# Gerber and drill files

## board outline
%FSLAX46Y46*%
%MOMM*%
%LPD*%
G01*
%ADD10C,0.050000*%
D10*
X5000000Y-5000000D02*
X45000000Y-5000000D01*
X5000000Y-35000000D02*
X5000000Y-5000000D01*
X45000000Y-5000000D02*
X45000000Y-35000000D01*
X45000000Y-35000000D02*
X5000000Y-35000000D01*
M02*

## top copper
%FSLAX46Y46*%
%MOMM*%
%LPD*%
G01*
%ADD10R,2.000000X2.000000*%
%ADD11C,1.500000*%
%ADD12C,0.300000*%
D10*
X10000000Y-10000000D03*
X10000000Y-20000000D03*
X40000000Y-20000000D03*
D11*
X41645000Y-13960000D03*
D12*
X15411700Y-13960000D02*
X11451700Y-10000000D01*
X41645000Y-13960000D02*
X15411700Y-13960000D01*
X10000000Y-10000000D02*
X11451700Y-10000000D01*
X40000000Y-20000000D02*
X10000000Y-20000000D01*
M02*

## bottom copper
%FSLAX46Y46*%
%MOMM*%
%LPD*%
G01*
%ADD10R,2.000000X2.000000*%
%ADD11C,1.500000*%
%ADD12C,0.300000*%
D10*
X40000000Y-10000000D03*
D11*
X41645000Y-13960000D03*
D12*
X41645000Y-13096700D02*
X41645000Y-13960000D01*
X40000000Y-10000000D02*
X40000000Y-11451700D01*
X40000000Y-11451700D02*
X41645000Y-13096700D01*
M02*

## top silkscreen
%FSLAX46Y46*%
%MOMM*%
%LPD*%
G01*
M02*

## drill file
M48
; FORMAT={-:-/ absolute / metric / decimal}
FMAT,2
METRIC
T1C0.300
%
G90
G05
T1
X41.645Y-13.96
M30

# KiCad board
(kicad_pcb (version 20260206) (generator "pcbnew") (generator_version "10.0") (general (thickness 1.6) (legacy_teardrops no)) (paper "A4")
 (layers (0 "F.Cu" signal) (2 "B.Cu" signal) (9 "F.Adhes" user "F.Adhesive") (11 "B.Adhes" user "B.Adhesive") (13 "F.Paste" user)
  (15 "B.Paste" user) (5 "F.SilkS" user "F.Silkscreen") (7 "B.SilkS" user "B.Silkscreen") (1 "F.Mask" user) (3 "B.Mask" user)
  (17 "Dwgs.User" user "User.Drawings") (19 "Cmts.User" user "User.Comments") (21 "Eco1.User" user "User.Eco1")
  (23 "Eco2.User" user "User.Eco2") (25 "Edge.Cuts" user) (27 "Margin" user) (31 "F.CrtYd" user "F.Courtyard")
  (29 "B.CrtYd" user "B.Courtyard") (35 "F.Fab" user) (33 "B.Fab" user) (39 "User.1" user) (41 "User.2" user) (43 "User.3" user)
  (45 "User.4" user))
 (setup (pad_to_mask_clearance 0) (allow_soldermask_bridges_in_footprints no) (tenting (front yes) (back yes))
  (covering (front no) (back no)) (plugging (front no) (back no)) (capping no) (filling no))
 (gr_line (start 5 5) (end 45 5) (stroke (width 0.05) (type default)) (layer "Edge.Cuts"))
 (gr_line (start 5 35) (end 5 5) (stroke (width 0.05) (type default)) (layer "Edge.Cuts"))
 (gr_line (start 45 5) (end 45 35) (stroke (width 0.05) (type default)) (layer "Edge.Cuts"))
 (gr_line (start 45 35) (end 5 35) (stroke (width 0.05) (type default)) (layer "Edge.Cuts"))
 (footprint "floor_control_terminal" (layer "F.Cu") (at 10 10)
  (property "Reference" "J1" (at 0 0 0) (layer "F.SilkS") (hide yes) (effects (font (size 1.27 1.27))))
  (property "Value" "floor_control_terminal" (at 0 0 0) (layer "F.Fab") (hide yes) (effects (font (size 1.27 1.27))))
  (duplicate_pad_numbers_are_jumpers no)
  (pad "1" smd rect (at 0 0) (size 2 2) (layers "F.Cu" "F.Paste" "F.Mask") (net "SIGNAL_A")))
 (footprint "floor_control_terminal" (layer "B.Cu") (at 40 10)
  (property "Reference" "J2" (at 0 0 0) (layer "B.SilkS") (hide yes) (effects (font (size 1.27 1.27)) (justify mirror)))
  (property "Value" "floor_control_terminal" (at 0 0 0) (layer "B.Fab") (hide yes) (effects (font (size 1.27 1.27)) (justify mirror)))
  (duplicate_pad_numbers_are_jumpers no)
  (pad "1" smd rect (at 0 0) (size 2 2) (layers "B.Cu" "B.Paste" "B.Mask") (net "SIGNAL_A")))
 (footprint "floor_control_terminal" (layer "F.Cu") (at 10 20)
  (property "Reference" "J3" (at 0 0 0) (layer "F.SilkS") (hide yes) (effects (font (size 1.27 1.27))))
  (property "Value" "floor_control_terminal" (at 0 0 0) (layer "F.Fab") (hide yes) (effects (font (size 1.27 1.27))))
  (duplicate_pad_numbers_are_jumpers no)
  (pad "1" smd rect (at 0 0) (size 2 2) (layers "F.Cu" "F.Paste" "F.Mask") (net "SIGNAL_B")))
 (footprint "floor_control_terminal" (layer "F.Cu") (at 40 20)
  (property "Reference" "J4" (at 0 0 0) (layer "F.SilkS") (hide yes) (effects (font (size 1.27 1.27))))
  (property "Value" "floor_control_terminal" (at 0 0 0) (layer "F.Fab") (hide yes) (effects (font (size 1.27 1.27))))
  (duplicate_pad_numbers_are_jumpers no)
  (pad "1" smd rect (at 0 0) (size 2 2) (layers "F.Cu" "F.Paste" "F.Mask") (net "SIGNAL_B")))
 (segment (start 15.4117 13.96) (end 11.4517 10) (width 0.3) (layer "F.Cu") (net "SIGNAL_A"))
 (segment (start 41.645 13.96) (end 15.4117 13.96) (width 0.3) (layer "F.Cu") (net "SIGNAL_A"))
 (segment (start 10 10) (end 11.4517 10) (width 0.3) (layer "F.Cu") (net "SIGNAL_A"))
 (via (at 41.645 13.96) (size 1.5) (drill 0.3) (layers "F.Cu" "B.Cu") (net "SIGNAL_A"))
 (segment (start 41.645 13.0967) (end 41.645 13.96) (width 0.3) (layer "B.Cu") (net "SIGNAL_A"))
 (segment (start 40 10) (end 40 11.4517) (width 0.3) (layer "B.Cu") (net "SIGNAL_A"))
 (segment (start 40 11.4517) (end 41.645 13.0967) (width 0.3) (layer "B.Cu") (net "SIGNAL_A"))
 (segment (start 40 20) (end 10 20) (width 0.3) (layer "F.Cu") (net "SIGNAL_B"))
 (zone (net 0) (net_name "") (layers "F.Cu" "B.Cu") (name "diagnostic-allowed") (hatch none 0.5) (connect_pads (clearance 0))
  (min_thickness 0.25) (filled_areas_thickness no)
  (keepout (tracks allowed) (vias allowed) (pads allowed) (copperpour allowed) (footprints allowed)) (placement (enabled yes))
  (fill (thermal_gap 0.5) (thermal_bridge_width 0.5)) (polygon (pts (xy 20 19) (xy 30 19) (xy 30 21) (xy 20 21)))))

